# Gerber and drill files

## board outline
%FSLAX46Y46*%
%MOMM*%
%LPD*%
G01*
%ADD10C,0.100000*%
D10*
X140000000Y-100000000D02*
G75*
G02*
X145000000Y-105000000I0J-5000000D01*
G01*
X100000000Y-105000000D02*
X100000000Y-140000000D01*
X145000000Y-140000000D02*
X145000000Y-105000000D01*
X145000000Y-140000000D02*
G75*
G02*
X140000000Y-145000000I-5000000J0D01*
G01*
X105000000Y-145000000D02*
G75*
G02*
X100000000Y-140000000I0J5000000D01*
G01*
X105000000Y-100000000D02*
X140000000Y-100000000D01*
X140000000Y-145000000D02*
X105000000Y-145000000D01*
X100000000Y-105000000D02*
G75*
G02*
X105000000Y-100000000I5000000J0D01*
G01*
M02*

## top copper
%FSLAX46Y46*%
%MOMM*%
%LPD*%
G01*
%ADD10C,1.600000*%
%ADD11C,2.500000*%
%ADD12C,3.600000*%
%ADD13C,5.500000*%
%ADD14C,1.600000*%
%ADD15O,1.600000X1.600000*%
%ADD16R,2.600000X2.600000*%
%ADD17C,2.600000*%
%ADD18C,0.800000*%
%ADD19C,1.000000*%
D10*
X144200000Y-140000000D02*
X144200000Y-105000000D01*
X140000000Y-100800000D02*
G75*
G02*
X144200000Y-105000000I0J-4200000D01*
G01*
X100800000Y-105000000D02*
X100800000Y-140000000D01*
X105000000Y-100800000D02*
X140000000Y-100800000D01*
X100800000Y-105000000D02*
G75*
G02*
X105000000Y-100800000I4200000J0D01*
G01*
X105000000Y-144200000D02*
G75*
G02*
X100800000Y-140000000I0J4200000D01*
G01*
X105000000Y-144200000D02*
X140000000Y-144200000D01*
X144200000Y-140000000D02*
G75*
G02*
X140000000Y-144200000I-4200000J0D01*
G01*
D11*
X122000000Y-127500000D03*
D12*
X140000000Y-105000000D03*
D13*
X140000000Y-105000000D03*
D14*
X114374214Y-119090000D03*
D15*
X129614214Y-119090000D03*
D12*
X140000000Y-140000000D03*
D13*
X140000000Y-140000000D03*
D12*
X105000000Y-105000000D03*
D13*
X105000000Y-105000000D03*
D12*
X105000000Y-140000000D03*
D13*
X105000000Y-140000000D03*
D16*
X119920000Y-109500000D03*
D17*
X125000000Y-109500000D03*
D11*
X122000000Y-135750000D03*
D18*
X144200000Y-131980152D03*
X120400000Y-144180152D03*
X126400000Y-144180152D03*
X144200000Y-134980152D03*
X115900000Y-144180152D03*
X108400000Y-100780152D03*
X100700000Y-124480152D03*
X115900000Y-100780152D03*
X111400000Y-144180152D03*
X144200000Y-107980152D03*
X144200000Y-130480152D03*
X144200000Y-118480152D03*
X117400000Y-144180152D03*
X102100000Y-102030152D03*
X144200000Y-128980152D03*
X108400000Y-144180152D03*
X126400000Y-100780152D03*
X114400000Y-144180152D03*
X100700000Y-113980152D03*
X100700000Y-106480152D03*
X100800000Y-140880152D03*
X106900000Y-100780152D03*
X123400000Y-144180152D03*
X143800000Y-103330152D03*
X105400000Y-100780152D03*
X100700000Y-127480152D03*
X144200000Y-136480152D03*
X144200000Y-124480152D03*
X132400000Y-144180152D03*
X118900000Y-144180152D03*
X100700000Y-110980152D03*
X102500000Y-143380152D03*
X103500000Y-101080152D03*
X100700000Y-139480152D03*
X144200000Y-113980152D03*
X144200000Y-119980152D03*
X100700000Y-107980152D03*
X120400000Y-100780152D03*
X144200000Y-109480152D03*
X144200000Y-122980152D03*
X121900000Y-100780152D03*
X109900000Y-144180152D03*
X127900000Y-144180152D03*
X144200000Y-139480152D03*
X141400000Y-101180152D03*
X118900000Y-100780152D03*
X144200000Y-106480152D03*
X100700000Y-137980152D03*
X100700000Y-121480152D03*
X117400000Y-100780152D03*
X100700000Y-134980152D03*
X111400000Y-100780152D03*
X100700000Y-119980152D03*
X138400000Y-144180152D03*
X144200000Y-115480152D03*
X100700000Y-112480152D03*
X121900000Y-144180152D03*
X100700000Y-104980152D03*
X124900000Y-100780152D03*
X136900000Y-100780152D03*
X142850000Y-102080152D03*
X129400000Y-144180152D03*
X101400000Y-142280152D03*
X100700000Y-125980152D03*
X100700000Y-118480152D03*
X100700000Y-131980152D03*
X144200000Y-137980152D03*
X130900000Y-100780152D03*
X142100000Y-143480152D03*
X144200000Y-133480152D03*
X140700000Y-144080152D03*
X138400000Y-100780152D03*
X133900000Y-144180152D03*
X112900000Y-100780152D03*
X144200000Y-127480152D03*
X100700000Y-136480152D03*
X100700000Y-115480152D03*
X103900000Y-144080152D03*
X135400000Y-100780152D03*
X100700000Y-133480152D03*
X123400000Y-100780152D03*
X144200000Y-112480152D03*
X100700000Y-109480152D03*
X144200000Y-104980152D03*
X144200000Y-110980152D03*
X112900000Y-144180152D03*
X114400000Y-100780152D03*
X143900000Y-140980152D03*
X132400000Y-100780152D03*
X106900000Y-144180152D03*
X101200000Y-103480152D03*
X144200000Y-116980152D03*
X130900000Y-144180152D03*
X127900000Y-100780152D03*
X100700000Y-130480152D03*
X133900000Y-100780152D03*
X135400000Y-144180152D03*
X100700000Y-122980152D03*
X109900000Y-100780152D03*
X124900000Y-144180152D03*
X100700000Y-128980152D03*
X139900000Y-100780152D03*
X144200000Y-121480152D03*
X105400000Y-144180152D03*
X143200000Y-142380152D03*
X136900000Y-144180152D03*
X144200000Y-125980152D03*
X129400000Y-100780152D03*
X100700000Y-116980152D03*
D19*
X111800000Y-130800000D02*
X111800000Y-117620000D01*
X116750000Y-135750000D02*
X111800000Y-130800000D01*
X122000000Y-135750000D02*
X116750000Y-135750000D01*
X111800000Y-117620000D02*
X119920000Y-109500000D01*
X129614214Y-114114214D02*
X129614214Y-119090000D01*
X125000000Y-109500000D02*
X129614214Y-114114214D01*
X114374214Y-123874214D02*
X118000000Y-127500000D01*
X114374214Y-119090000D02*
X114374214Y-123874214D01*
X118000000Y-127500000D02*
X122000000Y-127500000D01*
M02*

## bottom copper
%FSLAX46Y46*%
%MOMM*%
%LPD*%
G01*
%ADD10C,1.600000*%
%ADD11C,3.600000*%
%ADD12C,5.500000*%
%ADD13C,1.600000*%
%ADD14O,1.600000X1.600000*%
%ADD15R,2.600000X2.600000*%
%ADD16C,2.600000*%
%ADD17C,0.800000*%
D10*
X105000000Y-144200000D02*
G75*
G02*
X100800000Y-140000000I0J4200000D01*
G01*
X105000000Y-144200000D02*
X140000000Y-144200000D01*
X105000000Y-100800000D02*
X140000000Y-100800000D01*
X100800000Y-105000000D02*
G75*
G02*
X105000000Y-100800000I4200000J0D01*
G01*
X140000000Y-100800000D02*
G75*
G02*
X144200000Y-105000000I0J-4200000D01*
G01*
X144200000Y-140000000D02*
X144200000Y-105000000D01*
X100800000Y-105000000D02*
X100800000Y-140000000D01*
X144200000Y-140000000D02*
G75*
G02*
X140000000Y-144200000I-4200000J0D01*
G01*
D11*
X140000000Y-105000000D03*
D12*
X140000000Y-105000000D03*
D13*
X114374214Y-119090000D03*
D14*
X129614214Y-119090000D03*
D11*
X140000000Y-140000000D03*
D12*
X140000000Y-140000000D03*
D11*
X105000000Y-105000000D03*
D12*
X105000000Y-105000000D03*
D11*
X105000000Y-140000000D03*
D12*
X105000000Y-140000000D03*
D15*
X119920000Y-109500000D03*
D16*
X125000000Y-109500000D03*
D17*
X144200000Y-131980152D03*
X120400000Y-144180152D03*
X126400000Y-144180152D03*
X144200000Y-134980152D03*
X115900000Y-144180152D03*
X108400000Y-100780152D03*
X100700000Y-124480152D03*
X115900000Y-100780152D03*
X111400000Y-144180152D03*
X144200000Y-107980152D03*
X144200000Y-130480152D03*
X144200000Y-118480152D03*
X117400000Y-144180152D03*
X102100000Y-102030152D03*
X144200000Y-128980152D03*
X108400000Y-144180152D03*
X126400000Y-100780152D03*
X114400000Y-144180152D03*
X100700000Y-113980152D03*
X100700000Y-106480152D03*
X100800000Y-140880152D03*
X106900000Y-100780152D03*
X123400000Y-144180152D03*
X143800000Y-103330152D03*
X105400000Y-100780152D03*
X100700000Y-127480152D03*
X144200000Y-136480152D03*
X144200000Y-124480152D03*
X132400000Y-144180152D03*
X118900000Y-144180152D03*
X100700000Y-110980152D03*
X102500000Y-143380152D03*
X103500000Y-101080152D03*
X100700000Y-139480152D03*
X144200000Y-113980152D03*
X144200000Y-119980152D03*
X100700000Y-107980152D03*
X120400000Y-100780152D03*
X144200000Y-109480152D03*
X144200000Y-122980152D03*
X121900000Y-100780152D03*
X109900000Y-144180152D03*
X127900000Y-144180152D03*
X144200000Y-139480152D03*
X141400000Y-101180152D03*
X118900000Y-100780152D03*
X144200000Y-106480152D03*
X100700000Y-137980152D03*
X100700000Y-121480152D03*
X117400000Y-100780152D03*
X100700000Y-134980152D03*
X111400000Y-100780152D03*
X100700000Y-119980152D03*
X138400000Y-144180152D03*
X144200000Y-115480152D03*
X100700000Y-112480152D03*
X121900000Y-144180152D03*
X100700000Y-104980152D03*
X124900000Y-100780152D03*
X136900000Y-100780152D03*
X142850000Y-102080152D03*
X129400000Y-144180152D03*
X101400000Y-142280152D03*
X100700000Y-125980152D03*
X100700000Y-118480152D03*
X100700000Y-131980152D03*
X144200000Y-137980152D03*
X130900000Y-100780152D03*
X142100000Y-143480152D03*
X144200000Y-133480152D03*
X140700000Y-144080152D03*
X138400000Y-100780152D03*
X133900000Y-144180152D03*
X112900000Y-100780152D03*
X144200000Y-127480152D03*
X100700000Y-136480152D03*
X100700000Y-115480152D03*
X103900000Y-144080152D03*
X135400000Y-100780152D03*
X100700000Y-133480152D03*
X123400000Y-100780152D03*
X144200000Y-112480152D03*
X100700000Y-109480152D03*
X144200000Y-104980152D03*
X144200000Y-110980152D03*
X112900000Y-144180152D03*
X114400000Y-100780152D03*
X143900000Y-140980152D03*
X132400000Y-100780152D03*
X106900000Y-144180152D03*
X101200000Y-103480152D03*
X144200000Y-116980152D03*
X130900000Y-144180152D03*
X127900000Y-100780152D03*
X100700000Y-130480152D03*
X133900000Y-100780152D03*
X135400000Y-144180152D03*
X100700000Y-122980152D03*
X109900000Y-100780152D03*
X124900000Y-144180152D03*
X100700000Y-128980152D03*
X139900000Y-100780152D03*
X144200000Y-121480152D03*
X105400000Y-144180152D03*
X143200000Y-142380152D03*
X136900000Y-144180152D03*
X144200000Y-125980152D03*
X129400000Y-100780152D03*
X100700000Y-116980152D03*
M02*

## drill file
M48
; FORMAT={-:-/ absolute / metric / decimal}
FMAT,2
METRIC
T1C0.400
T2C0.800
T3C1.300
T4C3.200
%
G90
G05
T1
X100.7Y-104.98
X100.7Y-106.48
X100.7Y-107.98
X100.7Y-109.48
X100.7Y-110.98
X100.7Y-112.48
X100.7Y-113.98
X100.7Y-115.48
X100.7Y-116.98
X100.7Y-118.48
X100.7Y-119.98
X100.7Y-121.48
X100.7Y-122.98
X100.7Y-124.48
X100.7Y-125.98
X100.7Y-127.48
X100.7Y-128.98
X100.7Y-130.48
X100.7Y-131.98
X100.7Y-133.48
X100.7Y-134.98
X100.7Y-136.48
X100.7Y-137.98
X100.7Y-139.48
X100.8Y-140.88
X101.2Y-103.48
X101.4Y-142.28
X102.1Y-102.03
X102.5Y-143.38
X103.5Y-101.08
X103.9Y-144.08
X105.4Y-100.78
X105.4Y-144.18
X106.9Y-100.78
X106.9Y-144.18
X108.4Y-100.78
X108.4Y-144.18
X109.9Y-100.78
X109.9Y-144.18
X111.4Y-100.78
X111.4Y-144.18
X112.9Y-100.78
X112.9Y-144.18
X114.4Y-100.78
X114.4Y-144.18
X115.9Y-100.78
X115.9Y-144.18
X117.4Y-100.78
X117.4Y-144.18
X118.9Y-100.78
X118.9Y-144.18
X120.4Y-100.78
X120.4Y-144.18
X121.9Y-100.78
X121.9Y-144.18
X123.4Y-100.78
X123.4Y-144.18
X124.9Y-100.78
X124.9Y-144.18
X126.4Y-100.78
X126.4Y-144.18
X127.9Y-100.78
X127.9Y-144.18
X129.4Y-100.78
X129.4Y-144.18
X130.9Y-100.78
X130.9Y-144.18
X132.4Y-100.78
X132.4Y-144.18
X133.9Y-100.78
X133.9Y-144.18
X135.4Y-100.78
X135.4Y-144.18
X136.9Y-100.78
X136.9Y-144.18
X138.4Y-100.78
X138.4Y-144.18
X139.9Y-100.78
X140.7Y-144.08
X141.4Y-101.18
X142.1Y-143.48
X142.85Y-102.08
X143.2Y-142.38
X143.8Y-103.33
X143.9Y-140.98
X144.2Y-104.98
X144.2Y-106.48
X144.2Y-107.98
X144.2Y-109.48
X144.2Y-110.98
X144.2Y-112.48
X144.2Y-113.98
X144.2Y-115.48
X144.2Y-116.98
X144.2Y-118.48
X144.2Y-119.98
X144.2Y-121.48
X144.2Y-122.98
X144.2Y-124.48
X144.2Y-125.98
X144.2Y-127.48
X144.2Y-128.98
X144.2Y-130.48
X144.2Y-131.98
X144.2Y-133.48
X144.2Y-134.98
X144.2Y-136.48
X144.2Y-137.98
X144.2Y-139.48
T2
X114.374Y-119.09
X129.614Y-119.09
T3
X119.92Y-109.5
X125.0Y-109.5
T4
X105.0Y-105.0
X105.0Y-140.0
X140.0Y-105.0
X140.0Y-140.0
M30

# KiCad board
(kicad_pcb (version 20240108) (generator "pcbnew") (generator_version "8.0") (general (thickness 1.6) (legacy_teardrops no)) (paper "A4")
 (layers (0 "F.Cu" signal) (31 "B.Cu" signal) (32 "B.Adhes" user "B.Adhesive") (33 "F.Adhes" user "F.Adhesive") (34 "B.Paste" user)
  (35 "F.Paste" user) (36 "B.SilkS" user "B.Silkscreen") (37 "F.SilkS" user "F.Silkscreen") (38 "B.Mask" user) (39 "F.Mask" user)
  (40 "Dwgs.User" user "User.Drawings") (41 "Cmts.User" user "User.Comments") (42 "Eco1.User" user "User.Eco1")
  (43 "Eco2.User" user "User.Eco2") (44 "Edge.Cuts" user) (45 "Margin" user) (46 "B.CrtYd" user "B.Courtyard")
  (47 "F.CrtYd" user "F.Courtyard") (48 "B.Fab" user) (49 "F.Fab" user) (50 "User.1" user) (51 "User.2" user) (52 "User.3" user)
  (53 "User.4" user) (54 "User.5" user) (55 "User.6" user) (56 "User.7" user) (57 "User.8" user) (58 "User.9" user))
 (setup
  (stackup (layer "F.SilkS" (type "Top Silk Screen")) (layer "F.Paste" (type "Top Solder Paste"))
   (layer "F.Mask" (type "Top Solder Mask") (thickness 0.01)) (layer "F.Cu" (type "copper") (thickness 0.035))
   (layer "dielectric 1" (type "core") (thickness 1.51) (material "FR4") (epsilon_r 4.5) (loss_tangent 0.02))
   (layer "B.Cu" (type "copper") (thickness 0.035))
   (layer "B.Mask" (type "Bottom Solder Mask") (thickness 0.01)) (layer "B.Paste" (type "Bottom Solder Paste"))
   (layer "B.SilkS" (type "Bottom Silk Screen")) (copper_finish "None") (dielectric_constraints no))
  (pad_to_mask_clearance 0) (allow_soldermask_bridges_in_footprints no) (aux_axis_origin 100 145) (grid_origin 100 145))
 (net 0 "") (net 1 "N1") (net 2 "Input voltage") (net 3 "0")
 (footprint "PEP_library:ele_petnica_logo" (layer "F.Cu") (at 136 126.6)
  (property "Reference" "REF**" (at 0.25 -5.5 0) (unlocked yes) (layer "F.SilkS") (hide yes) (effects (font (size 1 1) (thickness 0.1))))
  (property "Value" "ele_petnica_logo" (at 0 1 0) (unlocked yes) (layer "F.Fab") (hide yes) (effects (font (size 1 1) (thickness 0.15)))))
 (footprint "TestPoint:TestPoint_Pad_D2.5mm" (layer "F.Cu") (at 122 127.5)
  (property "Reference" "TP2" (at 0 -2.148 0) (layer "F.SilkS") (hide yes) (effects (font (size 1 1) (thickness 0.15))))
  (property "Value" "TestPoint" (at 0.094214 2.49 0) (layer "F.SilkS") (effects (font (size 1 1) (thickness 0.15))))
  (pad "1" smd circle (at 0 0) (size 2.5 2.5) (layers "F.Cu" "F.Mask") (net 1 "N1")))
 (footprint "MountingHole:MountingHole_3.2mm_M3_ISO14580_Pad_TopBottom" (layer "F.Cu") (at 140 105)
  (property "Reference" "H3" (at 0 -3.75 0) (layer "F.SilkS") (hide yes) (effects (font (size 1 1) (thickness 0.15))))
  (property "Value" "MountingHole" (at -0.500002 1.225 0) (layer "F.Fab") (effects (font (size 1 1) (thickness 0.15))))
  (pad "1" thru_hole circle (at 0 0) (size 3.6 3.6) (drill 3.2) (layers "*.Cu" "*.Mask") (remove_unused_layers no))
  (pad "1" connect circle (at 0 0) (size 5.5 5.5) (layers "F.Cu" "F.Mask"))
  (pad "1" connect circle (at 0 0) (size 5.5 5.5) (layers "B.Cu" "B.Mask")))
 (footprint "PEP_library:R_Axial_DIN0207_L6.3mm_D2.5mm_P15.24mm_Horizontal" (layer "F.Cu") (at 114.374214 119.09)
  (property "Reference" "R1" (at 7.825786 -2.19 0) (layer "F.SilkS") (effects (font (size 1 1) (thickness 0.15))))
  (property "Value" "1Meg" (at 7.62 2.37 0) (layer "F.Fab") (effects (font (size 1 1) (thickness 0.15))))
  (pad "1" thru_hole circle (at 0 0) (size 1.6 1.6) (drill 0.8) (layers "*.Cu" "*.Mask") (remove_unused_layers no) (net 1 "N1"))
  (pad "2" thru_hole oval (at 15.24 0) (size 1.6 1.6) (drill 0.8) (layers "*.Cu" "*.Mask") (remove_unused_layers no) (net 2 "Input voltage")))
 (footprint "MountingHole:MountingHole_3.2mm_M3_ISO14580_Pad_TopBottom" (layer "F.Cu") (at 140 140)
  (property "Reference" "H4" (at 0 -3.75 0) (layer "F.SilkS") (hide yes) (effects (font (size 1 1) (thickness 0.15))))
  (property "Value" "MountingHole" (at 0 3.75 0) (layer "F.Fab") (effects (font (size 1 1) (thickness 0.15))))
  (pad "1" thru_hole circle (at 0 0) (size 3.6 3.6) (drill 3.2) (layers "*.Cu" "*.Mask") (remove_unused_layers no))
  (pad "1" connect circle (at 0 0) (size 5.5 5.5) (layers "F.Cu" "F.Mask"))
  (pad "1" connect circle (at 0 0) (size 5.5 5.5) (layers "B.Cu" "B.Mask")))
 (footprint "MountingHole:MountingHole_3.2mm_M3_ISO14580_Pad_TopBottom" (layer "F.Cu") (at 105 105)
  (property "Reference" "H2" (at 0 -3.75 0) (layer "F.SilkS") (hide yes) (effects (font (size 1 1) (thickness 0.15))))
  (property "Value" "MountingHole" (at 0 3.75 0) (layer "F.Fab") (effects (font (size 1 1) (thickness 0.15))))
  (pad "1" thru_hole circle (at 0 0) (size 3.6 3.6) (drill 3.2) (layers "*.Cu" "*.Mask") (remove_unused_layers no))
  (pad "1" connect circle (at 0 0) (size 5.5 5.5) (layers "F.Cu" "F.Mask"))
  (pad "1" connect circle (at 0 0) (size 5.5 5.5) (layers "B.Cu" "B.Mask")))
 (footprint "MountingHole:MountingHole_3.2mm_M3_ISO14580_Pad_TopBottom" (layer "F.Cu") (at 105 140 -90)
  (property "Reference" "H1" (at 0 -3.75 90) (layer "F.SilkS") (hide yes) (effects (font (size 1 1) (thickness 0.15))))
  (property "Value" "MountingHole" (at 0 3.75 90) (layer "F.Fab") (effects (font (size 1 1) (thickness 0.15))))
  (pad "1" thru_hole circle (at 0 0 270) (size 3.6 3.6) (drill 3.2) (layers "*.Cu" "*.Mask") (remove_unused_layers no))
  (pad "1" connect circle (at 0 0 270) (size 5.5 5.5) (layers "F.Cu" "F.Mask"))
  (pad "1" connect circle (at 0 0 270) (size 5.5 5.5) (layers "B.Cu" "B.Mask")))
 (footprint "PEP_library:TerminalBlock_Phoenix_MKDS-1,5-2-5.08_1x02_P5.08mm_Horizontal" (layer "F.Cu") (at 119.92 109.5)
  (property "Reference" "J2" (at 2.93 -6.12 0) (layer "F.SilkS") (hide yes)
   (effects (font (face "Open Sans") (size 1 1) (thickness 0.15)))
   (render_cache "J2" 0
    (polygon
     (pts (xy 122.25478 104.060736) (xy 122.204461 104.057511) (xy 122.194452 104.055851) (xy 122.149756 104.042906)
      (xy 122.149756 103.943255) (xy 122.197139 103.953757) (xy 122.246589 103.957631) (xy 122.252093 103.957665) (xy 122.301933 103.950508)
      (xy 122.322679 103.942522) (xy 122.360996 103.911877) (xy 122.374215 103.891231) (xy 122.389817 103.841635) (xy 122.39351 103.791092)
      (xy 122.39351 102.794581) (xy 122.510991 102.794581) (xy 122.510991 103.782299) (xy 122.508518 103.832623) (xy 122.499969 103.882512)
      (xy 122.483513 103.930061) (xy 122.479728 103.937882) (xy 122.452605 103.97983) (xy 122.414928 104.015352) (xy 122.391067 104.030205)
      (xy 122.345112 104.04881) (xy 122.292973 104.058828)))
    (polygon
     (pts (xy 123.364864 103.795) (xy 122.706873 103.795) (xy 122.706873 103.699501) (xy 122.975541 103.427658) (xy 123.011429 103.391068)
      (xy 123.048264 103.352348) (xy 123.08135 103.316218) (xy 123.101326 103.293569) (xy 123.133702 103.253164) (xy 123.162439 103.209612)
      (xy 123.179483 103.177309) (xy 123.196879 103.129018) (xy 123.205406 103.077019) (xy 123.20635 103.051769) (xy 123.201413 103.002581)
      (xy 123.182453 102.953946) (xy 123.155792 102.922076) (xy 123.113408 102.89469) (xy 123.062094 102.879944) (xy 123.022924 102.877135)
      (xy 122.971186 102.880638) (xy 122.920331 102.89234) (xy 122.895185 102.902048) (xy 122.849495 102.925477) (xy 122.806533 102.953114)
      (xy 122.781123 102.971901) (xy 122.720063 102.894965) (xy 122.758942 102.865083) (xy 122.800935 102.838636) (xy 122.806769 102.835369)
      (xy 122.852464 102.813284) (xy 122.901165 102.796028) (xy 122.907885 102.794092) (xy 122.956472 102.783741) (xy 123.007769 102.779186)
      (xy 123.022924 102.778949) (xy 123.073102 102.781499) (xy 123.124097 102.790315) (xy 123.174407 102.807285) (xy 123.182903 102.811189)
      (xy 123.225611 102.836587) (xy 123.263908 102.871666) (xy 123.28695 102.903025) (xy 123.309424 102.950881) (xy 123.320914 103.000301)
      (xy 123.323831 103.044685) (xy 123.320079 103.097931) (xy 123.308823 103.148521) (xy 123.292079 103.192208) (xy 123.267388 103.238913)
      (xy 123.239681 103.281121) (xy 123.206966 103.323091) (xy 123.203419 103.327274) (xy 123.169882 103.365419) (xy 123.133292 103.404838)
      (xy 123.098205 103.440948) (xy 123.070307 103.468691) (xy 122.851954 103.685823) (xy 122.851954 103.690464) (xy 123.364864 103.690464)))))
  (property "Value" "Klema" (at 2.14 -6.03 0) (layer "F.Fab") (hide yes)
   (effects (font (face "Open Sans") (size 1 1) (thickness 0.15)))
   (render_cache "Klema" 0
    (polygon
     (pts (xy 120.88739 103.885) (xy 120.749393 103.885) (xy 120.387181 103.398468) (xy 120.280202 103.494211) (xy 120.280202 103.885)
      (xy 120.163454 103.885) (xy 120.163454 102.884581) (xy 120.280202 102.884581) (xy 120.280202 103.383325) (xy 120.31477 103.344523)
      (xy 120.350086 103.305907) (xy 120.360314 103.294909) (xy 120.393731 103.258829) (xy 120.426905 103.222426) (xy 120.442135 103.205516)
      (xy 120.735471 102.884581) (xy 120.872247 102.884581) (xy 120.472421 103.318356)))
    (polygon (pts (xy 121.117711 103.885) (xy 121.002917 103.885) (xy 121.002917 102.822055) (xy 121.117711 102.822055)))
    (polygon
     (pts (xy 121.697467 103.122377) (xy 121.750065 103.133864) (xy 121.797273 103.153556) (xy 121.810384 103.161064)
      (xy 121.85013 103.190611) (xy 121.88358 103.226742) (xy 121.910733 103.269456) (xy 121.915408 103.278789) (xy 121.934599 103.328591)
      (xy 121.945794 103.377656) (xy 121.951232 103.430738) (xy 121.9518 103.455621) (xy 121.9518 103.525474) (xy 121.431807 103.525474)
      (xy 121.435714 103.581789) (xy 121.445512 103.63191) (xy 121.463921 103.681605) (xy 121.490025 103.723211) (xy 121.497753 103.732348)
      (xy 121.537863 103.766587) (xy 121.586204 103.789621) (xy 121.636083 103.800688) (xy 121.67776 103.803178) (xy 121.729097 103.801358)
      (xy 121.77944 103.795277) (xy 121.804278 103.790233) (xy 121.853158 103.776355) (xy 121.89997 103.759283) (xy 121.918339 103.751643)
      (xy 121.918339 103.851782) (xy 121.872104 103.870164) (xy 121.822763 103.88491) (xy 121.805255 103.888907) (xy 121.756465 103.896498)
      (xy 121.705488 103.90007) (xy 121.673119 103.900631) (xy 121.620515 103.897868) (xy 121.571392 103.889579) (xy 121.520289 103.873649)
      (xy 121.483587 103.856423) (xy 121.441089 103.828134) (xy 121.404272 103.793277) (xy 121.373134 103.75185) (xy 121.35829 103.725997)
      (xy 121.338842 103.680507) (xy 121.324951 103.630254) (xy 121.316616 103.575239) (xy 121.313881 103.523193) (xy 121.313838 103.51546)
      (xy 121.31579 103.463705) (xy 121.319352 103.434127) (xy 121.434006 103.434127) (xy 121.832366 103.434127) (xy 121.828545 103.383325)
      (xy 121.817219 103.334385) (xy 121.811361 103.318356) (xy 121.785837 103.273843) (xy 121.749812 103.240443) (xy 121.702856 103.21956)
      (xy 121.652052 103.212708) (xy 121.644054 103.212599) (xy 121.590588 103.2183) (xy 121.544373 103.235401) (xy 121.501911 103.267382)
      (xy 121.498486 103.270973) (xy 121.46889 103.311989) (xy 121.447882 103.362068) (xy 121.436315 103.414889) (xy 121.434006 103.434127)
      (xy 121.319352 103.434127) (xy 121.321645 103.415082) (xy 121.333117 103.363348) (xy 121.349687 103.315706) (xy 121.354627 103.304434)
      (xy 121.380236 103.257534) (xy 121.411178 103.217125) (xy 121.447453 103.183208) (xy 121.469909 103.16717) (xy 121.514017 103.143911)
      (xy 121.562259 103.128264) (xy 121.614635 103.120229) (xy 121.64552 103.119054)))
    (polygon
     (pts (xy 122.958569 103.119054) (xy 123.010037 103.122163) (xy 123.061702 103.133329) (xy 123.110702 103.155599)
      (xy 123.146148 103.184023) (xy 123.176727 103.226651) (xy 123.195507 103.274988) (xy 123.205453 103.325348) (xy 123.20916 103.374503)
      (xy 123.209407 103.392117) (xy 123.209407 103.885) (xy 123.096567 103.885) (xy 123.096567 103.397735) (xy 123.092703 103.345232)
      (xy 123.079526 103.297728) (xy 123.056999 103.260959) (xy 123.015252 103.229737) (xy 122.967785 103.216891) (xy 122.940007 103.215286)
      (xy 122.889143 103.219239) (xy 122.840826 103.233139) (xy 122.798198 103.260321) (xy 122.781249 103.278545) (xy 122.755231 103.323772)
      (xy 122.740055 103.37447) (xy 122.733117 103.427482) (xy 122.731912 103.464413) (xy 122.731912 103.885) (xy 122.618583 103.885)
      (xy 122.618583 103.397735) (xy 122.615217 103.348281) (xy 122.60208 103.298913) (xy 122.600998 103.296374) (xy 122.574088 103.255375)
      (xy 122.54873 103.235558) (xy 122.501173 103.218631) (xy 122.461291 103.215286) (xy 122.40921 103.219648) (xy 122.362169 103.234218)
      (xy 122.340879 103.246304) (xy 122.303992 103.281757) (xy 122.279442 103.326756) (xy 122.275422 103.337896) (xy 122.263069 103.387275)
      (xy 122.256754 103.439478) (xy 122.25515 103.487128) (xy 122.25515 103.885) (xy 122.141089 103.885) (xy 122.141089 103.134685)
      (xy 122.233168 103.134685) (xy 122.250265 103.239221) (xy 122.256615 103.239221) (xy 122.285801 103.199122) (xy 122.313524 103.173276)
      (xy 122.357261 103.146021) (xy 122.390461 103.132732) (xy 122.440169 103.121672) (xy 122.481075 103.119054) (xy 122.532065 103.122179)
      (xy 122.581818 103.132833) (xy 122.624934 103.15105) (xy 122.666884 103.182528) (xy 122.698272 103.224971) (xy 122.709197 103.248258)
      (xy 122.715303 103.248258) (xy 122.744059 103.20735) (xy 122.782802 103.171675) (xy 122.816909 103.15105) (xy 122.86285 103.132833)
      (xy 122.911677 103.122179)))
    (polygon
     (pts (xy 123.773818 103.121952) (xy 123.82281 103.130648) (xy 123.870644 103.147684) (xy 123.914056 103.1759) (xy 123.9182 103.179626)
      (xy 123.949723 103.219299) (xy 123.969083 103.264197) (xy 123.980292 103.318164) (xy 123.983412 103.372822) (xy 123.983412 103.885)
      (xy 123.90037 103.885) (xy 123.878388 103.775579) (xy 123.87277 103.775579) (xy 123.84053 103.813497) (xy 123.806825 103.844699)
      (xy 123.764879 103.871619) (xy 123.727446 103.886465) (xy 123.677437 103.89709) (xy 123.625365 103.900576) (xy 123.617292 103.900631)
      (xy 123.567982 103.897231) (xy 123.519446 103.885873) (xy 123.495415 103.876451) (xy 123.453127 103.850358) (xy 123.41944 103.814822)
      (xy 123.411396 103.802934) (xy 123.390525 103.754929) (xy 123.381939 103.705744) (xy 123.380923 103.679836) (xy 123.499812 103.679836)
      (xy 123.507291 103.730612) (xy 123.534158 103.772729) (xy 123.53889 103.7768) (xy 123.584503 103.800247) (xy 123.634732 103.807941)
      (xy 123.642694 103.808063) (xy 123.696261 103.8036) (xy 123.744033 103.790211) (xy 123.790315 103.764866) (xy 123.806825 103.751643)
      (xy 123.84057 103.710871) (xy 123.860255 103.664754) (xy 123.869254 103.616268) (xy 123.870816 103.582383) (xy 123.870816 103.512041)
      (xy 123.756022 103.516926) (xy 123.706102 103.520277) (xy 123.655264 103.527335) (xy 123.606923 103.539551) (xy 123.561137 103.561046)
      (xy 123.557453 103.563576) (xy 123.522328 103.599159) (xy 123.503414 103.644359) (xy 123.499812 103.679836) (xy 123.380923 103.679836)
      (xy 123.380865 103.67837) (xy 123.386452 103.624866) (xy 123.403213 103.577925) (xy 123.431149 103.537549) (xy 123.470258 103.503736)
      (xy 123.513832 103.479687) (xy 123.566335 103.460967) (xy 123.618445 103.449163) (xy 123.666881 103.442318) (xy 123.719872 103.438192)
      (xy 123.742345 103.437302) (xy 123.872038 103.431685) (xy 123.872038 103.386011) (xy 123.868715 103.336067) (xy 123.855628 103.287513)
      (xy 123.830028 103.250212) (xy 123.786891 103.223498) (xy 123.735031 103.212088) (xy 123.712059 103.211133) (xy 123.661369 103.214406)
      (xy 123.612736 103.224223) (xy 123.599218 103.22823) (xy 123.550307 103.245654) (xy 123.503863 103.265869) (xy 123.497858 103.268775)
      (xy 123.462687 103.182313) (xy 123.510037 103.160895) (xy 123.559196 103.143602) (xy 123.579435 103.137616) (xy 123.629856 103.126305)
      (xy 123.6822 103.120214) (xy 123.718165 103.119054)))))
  (pad "1" thru_hole rect (at 0 0) (size 2.6 2.6) (drill 1.3) (layers "*.Cu" "*.Mask") (remove_unused_layers no) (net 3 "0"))
  (pad "2" thru_hole circle (at 5.08 0) (size 2.6 2.6) (drill 1.3) (layers "*.Cu" "*.Mask") (remove_unused_layers no)
   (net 2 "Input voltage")))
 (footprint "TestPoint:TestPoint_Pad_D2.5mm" (layer "F.Cu") (at 122 135.75)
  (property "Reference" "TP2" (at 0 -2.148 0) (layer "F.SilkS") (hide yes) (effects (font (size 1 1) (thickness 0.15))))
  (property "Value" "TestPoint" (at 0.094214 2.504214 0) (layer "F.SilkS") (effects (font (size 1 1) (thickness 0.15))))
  (pad "2" smd circle (at 0 0) (size 2.5 2.5) (layers "F.Cu" "F.Mask") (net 3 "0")))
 (gr_line (start 144.2 140) (end 144.2 105) (locked yes) (stroke (width 1.6) (type default)) (layer "F.Cu"))
 (gr_arc (start 140 100.8) (mid 142.969848 102.030152) (end 144.2 105) (locked yes) (stroke (width 1.6) (type default)) (layer "F.Cu"))
 (gr_line (start 100.8 105) (end 100.8 140) (locked yes) (stroke (width 1.6) (type default)) (layer "F.Cu"))
 (gr_line (start 105 100.8) (end 140 100.8) (locked yes) (stroke (width 1.6) (type default)) (layer "F.Cu"))
 (gr_arc (start 100.8 105) (mid 102.030152 102.030152) (end 105 100.8) (locked yes) (stroke (width 1.6) (type default)) (layer "F.Cu"))
 (gr_arc (start 105 144.2) (mid 102.030152 142.969848) (end 100.8 140) (locked yes) (stroke (width 1.6) (type default)) (layer "F.Cu"))
 (gr_line (start 105 144.2) (end 140 144.2) (locked yes) (stroke (width 1.6) (type default)) (layer "F.Cu"))
 (gr_arc (start 144.2 140) (mid 142.969848 142.969848) (end 140 144.2) (locked yes) (stroke (width 1.6) (type default)) (layer "F.Cu"))
 (gr_arc (start 105 144.2) (mid 102.030154 142.969848) (end 100.8 140) (locked yes) (stroke (width 1.6) (type default)) (layer "B.Cu"))
 (gr_line (start 105 144.2) (end 140 144.2) (locked yes) (stroke (width 1.6) (type default)) (layer "B.Cu"))
 (gr_line (start 105 100.8) (end 140 100.8) (locked yes) (stroke (width 1.6) (type default)) (layer "B.Cu"))
 (gr_arc (start 100.8 105) (mid 102.030152 102.030152) (end 105 100.8) (locked yes) (stroke (width 1.6) (type default)) (layer "B.Cu"))
 (gr_arc (start 140 100.8) (mid 142.96985 102.030151) (end 144.2 105) (locked yes) (stroke (width 1.6) (type default)) (layer "B.Cu"))
 (gr_line (start 144.2 140) (end 144.2 105) (locked yes) (stroke (width 1.6) (type default)) (layer "B.Cu"))
 (gr_line (start 100.8 105) (end 100.8 140) (locked yes) (stroke (width 1.6) (type default)) (layer "B.Cu"))
 (gr_arc (start 144.2 140) (mid 142.969849 142.969849) (end 140 144.2) (locked yes) (stroke (width 1.6) (type default)) (layer "B.Cu"))
 (gr_arc (start 140 100) (mid 143.535534 101.464466) (end 145 105) (locked yes) (stroke (width 0.1) (type default)) (layer "Edge.Cuts"))
 (gr_line (start 100 105) (end 100 140) (locked yes) (stroke (width 0.1) (type default)) (layer "Edge.Cuts"))
 (gr_line (start 145 140) (end 145 105) (locked yes) (stroke (width 0.1) (type default)) (layer "Edge.Cuts"))
 (gr_arc (start 145 140) (mid 143.535534 143.535534) (end 140 145) (locked yes) (stroke (width 0.1) (type default)) (layer "Edge.Cuts"))
 (gr_arc (start 105 145) (mid 101.464466 143.535534) (end 100 140) (locked yes) (stroke (width 0.1) (type default)) (layer "Edge.Cuts"))
 (gr_line (start 105 100) (end 140 100) (locked yes) (stroke (width 0.1) (type default)) (layer "Edge.Cuts"))
 (gr_line (start 140 145) (end 105 145) (locked yes) (stroke (width 0.1) (type default)) (layer "Edge.Cuts"))
 (gr_arc (start 100 105) (mid 101.464466 101.464466) (end 105 100) (locked yes) (stroke (width 0.1) (type default)) (layer "Edge.Cuts"))
 (via (at 144.2 131.980152) (size 0.8) (drill 0.4) (layers "F.Cu" "B.Cu") (locked yes) (free yes) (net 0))
 (via (at 120.4 144.180152) (size 0.8) (drill 0.4) (layers "F.Cu" "B.Cu") (locked yes) (free yes) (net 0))
 (via (at 126.4 144.180152) (size 0.8) (drill 0.4) (layers "F.Cu" "B.Cu") (locked yes) (free yes) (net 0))
 (via (at 144.2 134.980152) (size 0.8) (drill 0.4) (layers "F.Cu" "B.Cu") (locked yes) (free yes) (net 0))
 (via (at 115.9 144.180152) (size 0.8) (drill 0.4) (layers "F.Cu" "B.Cu") (locked yes) (free yes) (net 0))
 (via (at 108.4 100.780152) (size 0.8) (drill 0.4) (layers "F.Cu" "B.Cu") (locked yes) (free yes) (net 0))
 (via (at 100.7 124.480152) (size 0.8) (drill 0.4) (layers "F.Cu" "B.Cu") (locked yes) (free yes) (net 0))
 (via (at 115.9 100.780152) (size 0.8) (drill 0.4) (layers "F.Cu" "B.Cu") (locked yes) (free yes) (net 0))
 (via (at 111.4 144.180152) (size 0.8) (drill 0.4) (layers "F.Cu" "B.Cu") (locked yes) (free yes) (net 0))
 (via (at 144.2 107.980152) (size 0.8) (drill 0.4) (layers "F.Cu" "B.Cu") (locked yes) (free yes) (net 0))
 (via (at 144.2 130.480152) (size 0.8) (drill 0.4) (layers "F.Cu" "B.Cu") (locked yes) (free yes) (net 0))
 (via (at 144.2 118.480152) (size 0.8) (drill 0.4) (layers "F.Cu" "B.Cu") (locked yes) (free yes) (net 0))
 (via (at 117.4 144.180152) (size 0.8) (drill 0.4) (layers "F.Cu" "B.Cu") (locked yes) (free yes) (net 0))
 (via (at 102.1 102.030152) (size 0.8) (drill 0.4) (layers "F.Cu" "B.Cu") (locked yes) (free yes) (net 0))
 (via (at 144.2 128.980152) (size 0.8) (drill 0.4) (layers "F.Cu" "B.Cu") (locked yes) (free yes) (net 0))
 (via (at 108.4 144.180152) (size 0.8) (drill 0.4) (layers "F.Cu" "B.Cu") (locked yes) (free yes) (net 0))
 (via (at 126.4 100.780152) (size 0.8) (drill 0.4) (layers "F.Cu" "B.Cu") (locked yes) (free yes) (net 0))
 (via (at 114.4 144.180152) (size 0.8) (drill 0.4) (layers "F.Cu" "B.Cu") (locked yes) (free yes) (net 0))
 (via (at 100.7 113.980152) (size 0.8) (drill 0.4) (layers "F.Cu" "B.Cu") (locked yes) (free yes) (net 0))
 (via (at 100.7 106.480152) (size 0.8) (drill 0.4) (layers "F.Cu" "B.Cu") (locked yes) (free yes) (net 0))
 (via (at 100.8 140.880152) (size 0.8) (drill 0.4) (layers "F.Cu" "B.Cu") (locked yes) (free yes) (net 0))
 (via (at 106.9 100.780152) (size 0.8) (drill 0.4) (layers "F.Cu" "B.Cu") (locked yes) (free yes) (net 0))
 (via (at 123.4 144.180152) (size 0.8) (drill 0.4) (layers "F.Cu" "B.Cu") (locked yes) (free yes) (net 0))
 (via (at 143.8 103.330152) (size 0.8) (drill 0.4) (layers "F.Cu" "B.Cu") (locked yes) (free yes) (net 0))
 (via (at 105.4 100.780152) (size 0.8) (drill 0.4) (layers "F.Cu" "B.Cu") (locked yes) (free yes) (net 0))
 (via (at 100.7 127.480152) (size 0.8) (drill 0.4) (layers "F.Cu" "B.Cu") (locked yes) (free yes) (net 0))
 (via (at 144.2 136.480152) (size 0.8) (drill 0.4) (layers "F.Cu" "B.Cu") (locked yes) (free yes) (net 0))
 (via (at 144.2 124.480152) (size 0.8) (drill 0.4) (layers "F.Cu" "B.Cu") (locked yes) (free yes) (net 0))
 (via (at 132.4 144.180152) (size 0.8) (drill 0.4) (layers "F.Cu" "B.Cu") (locked yes) (free yes) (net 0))
 (via (at 118.9 144.180152) (size 0.8) (drill 0.4) (layers "F.Cu" "B.Cu") (locked yes) (free yes) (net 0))
 (via (at 100.7 110.980152) (size 0.8) (drill 0.4) (layers "F.Cu" "B.Cu") (locked yes) (free yes) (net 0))
 (via (at 102.5 143.380152) (size 0.8) (drill 0.4) (layers "F.Cu" "B.Cu") (locked yes) (free yes) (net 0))
 (via (at 103.5 101.080152) (size 0.8) (drill 0.4) (layers "F.Cu" "B.Cu") (locked yes) (free yes) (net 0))
 (via (at 100.7 139.480152) (size 0.8) (drill 0.4) (layers "F.Cu" "B.Cu") (locked yes) (free yes) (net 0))
 (via (at 144.2 113.980152) (size 0.8) (drill 0.4) (layers "F.Cu" "B.Cu") (locked yes) (free yes) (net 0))
 (via (at 144.2 119.980152) (size 0.8) (drill 0.4) (layers "F.Cu" "B.Cu") (locked yes) (free yes) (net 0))
 (via (at 100.7 107.980152) (size 0.8) (drill 0.4) (layers "F.Cu" "B.Cu") (locked yes) (free yes) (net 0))
 (via (at 120.4 100.780152) (size 0.8) (drill 0.4) (layers "F.Cu" "B.Cu") (locked yes) (free yes) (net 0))
 (via (at 144.2 109.480152) (size 0.8) (drill 0.4) (layers "F.Cu" "B.Cu") (locked yes) (free yes) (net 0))
 (via (at 144.2 122.980152) (size 0.8) (drill 0.4) (layers "F.Cu" "B.Cu") (locked yes) (free yes) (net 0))
 (via (at 121.9 100.780152) (size 0.8) (drill 0.4) (layers "F.Cu" "B.Cu") (locked yes) (free yes) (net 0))
 (via (at 109.9 144.180152) (size 0.8) (drill 0.4) (layers "F.Cu" "B.Cu") (locked yes) (free yes) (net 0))
 (via (at 127.9 144.180152) (size 0.8) (drill 0.4) (layers "F.Cu" "B.Cu") (locked yes) (free yes) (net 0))
 (via (at 144.2 139.480152) (size 0.8) (drill 0.4) (layers "F.Cu" "B.Cu") (locked yes) (free yes) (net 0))
 (via (at 141.4 101.180152) (size 0.8) (drill 0.4) (layers "F.Cu" "B.Cu") (locked yes) (free yes) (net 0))
 (via (at 118.9 100.780152) (size 0.8) (drill 0.4) (layers "F.Cu" "B.Cu") (locked yes) (free yes) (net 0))
 (via (at 144.2 106.480152) (size 0.8) (drill 0.4) (layers "F.Cu" "B.Cu") (locked yes) (free yes) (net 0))
 (via (at 100.7 137.980152) (size 0.8) (drill 0.4) (layers "F.Cu" "B.Cu") (locked yes) (free yes) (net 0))
 (via (at 100.7 121.480152) (size 0.8) (drill 0.4) (layers "F.Cu" "B.Cu") (locked yes) (free yes) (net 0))
 (via (at 117.4 100.780152) (size 0.8) (drill 0.4) (layers "F.Cu" "B.Cu") (locked yes) (free yes) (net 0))
 (via (at 100.7 134.980152) (size 0.8) (drill 0.4) (layers "F.Cu" "B.Cu") (locked yes) (free yes) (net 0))
 (via (at 111.4 100.780152) (size 0.8) (drill 0.4) (layers "F.Cu" "B.Cu") (locked yes) (free yes) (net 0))
 (via (at 100.7 119.980152) (size 0.8) (drill 0.4) (layers "F.Cu" "B.Cu") (locked yes) (free yes) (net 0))
 (via (at 138.4 144.180152) (size 0.8) (drill 0.4) (layers "F.Cu" "B.Cu") (locked yes) (free yes) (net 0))
 (via (at 144.2 115.480152) (size 0.8) (drill 0.4) (layers "F.Cu" "B.Cu") (locked yes) (free yes) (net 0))
 (via (at 100.7 112.480152) (size 0.8) (drill 0.4) (layers "F.Cu" "B.Cu") (locked yes) (free yes) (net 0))
 (via (at 121.9 144.180152) (size 0.8) (drill 0.4) (layers "F.Cu" "B.Cu") (locked yes) (free yes) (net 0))
 (via (at 100.7 104.980152) (size 0.8) (drill 0.4) (layers "F.Cu" "B.Cu") (locked yes) (free yes) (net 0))
 (via (at 124.9 100.780152) (size 0.8) (drill 0.4) (layers "F.Cu" "B.Cu") (locked yes) (free yes) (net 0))
 (via (at 136.9 100.780152) (size 0.8) (drill 0.4) (layers "F.Cu" "B.Cu") (locked yes) (free yes) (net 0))
 (via (at 142.85 102.080152) (size 0.8) (drill 0.4) (layers "F.Cu" "B.Cu") (locked yes) (free yes) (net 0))
 (via (at 129.4 144.180152) (size 0.8) (drill 0.4) (layers "F.Cu" "B.Cu") (locked yes) (free yes) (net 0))
 (via (at 101.4 142.280152) (size 0.8) (drill 0.4) (layers "F.Cu" "B.Cu") (locked yes) (free yes) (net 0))
 (via (at 100.7 125.980152) (size 0.8) (drill 0.4) (layers "F.Cu" "B.Cu") (locked yes) (free yes) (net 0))
 (via (at 100.7 118.480152) (size 0.8) (drill 0.4) (layers "F.Cu" "B.Cu") (locked yes) (free yes) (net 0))
 (via (at 100.7 131.980152) (size 0.8) (drill 0.4) (layers "F.Cu" "B.Cu") (locked yes) (free yes) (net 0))
 (via (at 144.2 137.980152) (size 0.8) (drill 0.4) (layers "F.Cu" "B.Cu") (locked yes) (free yes) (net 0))
 (via (at 130.9 100.780152) (size 0.8) (drill 0.4) (layers "F.Cu" "B.Cu") (locked yes) (free yes) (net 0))
 (via (at 142.1 143.480152) (size 0.8) (drill 0.4) (layers "F.Cu" "B.Cu") (locked yes) (free yes) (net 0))
 (via (at 144.2 133.480152) (size 0.8) (drill 0.4) (layers "F.Cu" "B.Cu") (locked yes) (free yes) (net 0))
 (via (at 140.7 144.080152) (size 0.8) (drill 0.4) (layers "F.Cu" "B.Cu") (locked yes) (free yes) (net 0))
 (via (at 138.4 100.780152) (size 0.8) (drill 0.4) (layers "F.Cu" "B.Cu") (locked yes) (free yes) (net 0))
 (via (at 133.9 144.180152) (size 0.8) (drill 0.4) (layers "F.Cu" "B.Cu") (locked yes) (free yes) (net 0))
 (via (at 112.9 100.780152) (size 0.8) (drill 0.4) (layers "F.Cu" "B.Cu") (locked yes) (free yes) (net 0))
 (via (at 144.2 127.480152) (size 0.8) (drill 0.4) (layers "F.Cu" "B.Cu") (locked yes) (free yes) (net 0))
 (via (at 100.7 136.480152) (size 0.8) (drill 0.4) (layers "F.Cu" "B.Cu") (locked yes) (free yes) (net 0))
 (via (at 100.7 115.480152) (size 0.8) (drill 0.4) (layers "F.Cu" "B.Cu") (locked yes) (free yes) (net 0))
 (via (at 103.9 144.080152) (size 0.8) (drill 0.4) (layers "F.Cu" "B.Cu") (locked yes) (free yes) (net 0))
 (via (at 135.4 100.780152) (size 0.8) (drill 0.4) (layers "F.Cu" "B.Cu") (locked yes) (free yes) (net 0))
 (via (at 100.7 133.480152) (size 0.8) (drill 0.4) (layers "F.Cu" "B.Cu") (locked yes) (free yes) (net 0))
 (via (at 123.4 100.780152) (size 0.8) (drill 0.4) (layers "F.Cu" "B.Cu") (locked yes) (free yes) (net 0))
 (via (at 144.2 112.480152) (size 0.8) (drill 0.4) (layers "F.Cu" "B.Cu") (locked yes) (free yes) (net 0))
 (via (at 100.7 109.480152) (size 0.8) (drill 0.4) (layers "F.Cu" "B.Cu") (locked yes) (free yes) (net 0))
 (via (at 144.2 104.980152) (size 0.8) (drill 0.4) (layers "F.Cu" "B.Cu") (locked yes) (free yes) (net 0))
 (via (at 144.2 110.980152) (size 0.8) (drill 0.4) (layers "F.Cu" "B.Cu") (locked yes) (free yes) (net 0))
 (via (at 112.9 144.180152) (size 0.8) (drill 0.4) (layers "F.Cu" "B.Cu") (locked yes) (free yes) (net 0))
 (via (at 114.4 100.780152) (size 0.8) (drill 0.4) (layers "F.Cu" "B.Cu") (locked yes) (free yes) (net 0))
 (via (at 143.9 140.980152) (size 0.8) (drill 0.4) (layers "F.Cu" "B.Cu") (locked yes) (free yes) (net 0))
 (via (at 132.4 100.780152) (size 0.8) (drill 0.4) (layers "F.Cu" "B.Cu") (locked yes) (free yes) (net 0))
 (via (at 106.9 144.180152) (size 0.8) (drill 0.4) (layers "F.Cu" "B.Cu") (locked yes) (free yes) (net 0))
 (via (at 101.2 103.480152) (size 0.8) (drill 0.4) (layers "F.Cu" "B.Cu") (locked yes) (free yes) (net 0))
 (via (at 144.2 116.980152) (size 0.8) (drill 0.4) (layers "F.Cu" "B.Cu") (locked yes) (free yes) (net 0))
 (via (at 130.9 144.180152) (size 0.8) (drill 0.4) (layers "F.Cu" "B.Cu") (locked yes) (free yes) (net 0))
 (via (at 127.9 100.780152) (size 0.8) (drill 0.4) (layers "F.Cu" "B.Cu") (locked yes) (free yes) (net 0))
 (via (at 100.7 130.480152) (size 0.8) (drill 0.4) (layers "F.Cu" "B.Cu") (locked yes) (free yes) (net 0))
 (via (at 133.9 100.780152) (size 0.8) (drill 0.4) (layers "F.Cu" "B.Cu") (locked yes) (free yes) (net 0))
 (via (at 135.4 144.180152) (size 0.8) (drill 0.4) (layers "F.Cu" "B.Cu") (locked yes) (free yes) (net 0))
 (via (at 100.7 122.980152) (size 0.8) (drill 0.4) (layers "F.Cu" "B.Cu") (locked yes) (free yes) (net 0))
 (via (at 109.9 100.780152) (size 0.8) (drill 0.4) (layers "F.Cu" "B.Cu") (locked yes) (free yes) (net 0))
 (via (at 124.9 144.180152) (size 0.8) (drill 0.4) (layers "F.Cu" "B.Cu") (locked yes) (free yes) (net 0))
 (via (at 100.7 128.980152) (size 0.8) (drill 0.4) (layers "F.Cu" "B.Cu") (locked yes) (free yes) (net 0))
 (via (at 139.9 100.780152) (size 0.8) (drill 0.4) (layers "F.Cu" "B.Cu") (locked yes) (free yes) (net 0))
 (via (at 144.2 121.480152) (size 0.8) (drill 0.4) (layers "F.Cu" "B.Cu") (locked yes) (free yes) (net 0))
 (via (at 105.4 144.180152) (size 0.8) (drill 0.4) (layers "F.Cu" "B.Cu") (locked yes) (free yes) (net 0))
 (via (at 143.2 142.380152) (size 0.8) (drill 0.4) (layers "F.Cu" "B.Cu") (locked yes) (free yes) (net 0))
 (via (at 136.9 144.180152) (size 0.8) (drill 0.4) (layers "F.Cu" "B.Cu") (locked yes) (free yes) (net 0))
 (via (at 144.2 125.980152) (size 0.8) (drill 0.4) (layers "F.Cu" "B.Cu") (locked yes) (free yes) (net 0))
 (via (at 129.4 100.780152) (size 0.8) (drill 0.4) (layers "F.Cu" "B.Cu") (locked yes) (free yes) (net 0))
 (via (at 100.7 116.980152) (size 0.8) (drill 0.4) (layers "F.Cu" "B.Cu") (locked yes) (free yes) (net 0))
 (segment (start 111.8 130.8) (end 111.8 117.62) (width 1) (layer "F.Cu") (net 3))
 (segment (start 116.75 135.75) (end 111.8 130.8) (width 1) (layer "F.Cu") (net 3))
 (segment (start 122 135.75) (end 116.75 135.75) (width 1) (layer "F.Cu") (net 3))
 (segment (start 111.8 117.62) (end 119.92 109.5) (width 1) (layer "F.Cu") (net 3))
 (segment (start 129.614214 114.114214) (end 129.614214 119.09) (width 1) (layer "F.Cu") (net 2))
 (segment (start 125 109.5) (end 129.614214 114.114214) (width 1) (layer "F.Cu") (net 2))
 (segment (start 114.374214 123.874214) (end 118 127.5) (width 1) (layer "F.Cu") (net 1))
 (segment (start 114.374214 119.09) (end 114.374214 123.874214) (width 1) (layer "F.Cu") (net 1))
 (segment (start 118 127.5) (end 122 127.5) (width 1) (layer "F.Cu") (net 1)))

